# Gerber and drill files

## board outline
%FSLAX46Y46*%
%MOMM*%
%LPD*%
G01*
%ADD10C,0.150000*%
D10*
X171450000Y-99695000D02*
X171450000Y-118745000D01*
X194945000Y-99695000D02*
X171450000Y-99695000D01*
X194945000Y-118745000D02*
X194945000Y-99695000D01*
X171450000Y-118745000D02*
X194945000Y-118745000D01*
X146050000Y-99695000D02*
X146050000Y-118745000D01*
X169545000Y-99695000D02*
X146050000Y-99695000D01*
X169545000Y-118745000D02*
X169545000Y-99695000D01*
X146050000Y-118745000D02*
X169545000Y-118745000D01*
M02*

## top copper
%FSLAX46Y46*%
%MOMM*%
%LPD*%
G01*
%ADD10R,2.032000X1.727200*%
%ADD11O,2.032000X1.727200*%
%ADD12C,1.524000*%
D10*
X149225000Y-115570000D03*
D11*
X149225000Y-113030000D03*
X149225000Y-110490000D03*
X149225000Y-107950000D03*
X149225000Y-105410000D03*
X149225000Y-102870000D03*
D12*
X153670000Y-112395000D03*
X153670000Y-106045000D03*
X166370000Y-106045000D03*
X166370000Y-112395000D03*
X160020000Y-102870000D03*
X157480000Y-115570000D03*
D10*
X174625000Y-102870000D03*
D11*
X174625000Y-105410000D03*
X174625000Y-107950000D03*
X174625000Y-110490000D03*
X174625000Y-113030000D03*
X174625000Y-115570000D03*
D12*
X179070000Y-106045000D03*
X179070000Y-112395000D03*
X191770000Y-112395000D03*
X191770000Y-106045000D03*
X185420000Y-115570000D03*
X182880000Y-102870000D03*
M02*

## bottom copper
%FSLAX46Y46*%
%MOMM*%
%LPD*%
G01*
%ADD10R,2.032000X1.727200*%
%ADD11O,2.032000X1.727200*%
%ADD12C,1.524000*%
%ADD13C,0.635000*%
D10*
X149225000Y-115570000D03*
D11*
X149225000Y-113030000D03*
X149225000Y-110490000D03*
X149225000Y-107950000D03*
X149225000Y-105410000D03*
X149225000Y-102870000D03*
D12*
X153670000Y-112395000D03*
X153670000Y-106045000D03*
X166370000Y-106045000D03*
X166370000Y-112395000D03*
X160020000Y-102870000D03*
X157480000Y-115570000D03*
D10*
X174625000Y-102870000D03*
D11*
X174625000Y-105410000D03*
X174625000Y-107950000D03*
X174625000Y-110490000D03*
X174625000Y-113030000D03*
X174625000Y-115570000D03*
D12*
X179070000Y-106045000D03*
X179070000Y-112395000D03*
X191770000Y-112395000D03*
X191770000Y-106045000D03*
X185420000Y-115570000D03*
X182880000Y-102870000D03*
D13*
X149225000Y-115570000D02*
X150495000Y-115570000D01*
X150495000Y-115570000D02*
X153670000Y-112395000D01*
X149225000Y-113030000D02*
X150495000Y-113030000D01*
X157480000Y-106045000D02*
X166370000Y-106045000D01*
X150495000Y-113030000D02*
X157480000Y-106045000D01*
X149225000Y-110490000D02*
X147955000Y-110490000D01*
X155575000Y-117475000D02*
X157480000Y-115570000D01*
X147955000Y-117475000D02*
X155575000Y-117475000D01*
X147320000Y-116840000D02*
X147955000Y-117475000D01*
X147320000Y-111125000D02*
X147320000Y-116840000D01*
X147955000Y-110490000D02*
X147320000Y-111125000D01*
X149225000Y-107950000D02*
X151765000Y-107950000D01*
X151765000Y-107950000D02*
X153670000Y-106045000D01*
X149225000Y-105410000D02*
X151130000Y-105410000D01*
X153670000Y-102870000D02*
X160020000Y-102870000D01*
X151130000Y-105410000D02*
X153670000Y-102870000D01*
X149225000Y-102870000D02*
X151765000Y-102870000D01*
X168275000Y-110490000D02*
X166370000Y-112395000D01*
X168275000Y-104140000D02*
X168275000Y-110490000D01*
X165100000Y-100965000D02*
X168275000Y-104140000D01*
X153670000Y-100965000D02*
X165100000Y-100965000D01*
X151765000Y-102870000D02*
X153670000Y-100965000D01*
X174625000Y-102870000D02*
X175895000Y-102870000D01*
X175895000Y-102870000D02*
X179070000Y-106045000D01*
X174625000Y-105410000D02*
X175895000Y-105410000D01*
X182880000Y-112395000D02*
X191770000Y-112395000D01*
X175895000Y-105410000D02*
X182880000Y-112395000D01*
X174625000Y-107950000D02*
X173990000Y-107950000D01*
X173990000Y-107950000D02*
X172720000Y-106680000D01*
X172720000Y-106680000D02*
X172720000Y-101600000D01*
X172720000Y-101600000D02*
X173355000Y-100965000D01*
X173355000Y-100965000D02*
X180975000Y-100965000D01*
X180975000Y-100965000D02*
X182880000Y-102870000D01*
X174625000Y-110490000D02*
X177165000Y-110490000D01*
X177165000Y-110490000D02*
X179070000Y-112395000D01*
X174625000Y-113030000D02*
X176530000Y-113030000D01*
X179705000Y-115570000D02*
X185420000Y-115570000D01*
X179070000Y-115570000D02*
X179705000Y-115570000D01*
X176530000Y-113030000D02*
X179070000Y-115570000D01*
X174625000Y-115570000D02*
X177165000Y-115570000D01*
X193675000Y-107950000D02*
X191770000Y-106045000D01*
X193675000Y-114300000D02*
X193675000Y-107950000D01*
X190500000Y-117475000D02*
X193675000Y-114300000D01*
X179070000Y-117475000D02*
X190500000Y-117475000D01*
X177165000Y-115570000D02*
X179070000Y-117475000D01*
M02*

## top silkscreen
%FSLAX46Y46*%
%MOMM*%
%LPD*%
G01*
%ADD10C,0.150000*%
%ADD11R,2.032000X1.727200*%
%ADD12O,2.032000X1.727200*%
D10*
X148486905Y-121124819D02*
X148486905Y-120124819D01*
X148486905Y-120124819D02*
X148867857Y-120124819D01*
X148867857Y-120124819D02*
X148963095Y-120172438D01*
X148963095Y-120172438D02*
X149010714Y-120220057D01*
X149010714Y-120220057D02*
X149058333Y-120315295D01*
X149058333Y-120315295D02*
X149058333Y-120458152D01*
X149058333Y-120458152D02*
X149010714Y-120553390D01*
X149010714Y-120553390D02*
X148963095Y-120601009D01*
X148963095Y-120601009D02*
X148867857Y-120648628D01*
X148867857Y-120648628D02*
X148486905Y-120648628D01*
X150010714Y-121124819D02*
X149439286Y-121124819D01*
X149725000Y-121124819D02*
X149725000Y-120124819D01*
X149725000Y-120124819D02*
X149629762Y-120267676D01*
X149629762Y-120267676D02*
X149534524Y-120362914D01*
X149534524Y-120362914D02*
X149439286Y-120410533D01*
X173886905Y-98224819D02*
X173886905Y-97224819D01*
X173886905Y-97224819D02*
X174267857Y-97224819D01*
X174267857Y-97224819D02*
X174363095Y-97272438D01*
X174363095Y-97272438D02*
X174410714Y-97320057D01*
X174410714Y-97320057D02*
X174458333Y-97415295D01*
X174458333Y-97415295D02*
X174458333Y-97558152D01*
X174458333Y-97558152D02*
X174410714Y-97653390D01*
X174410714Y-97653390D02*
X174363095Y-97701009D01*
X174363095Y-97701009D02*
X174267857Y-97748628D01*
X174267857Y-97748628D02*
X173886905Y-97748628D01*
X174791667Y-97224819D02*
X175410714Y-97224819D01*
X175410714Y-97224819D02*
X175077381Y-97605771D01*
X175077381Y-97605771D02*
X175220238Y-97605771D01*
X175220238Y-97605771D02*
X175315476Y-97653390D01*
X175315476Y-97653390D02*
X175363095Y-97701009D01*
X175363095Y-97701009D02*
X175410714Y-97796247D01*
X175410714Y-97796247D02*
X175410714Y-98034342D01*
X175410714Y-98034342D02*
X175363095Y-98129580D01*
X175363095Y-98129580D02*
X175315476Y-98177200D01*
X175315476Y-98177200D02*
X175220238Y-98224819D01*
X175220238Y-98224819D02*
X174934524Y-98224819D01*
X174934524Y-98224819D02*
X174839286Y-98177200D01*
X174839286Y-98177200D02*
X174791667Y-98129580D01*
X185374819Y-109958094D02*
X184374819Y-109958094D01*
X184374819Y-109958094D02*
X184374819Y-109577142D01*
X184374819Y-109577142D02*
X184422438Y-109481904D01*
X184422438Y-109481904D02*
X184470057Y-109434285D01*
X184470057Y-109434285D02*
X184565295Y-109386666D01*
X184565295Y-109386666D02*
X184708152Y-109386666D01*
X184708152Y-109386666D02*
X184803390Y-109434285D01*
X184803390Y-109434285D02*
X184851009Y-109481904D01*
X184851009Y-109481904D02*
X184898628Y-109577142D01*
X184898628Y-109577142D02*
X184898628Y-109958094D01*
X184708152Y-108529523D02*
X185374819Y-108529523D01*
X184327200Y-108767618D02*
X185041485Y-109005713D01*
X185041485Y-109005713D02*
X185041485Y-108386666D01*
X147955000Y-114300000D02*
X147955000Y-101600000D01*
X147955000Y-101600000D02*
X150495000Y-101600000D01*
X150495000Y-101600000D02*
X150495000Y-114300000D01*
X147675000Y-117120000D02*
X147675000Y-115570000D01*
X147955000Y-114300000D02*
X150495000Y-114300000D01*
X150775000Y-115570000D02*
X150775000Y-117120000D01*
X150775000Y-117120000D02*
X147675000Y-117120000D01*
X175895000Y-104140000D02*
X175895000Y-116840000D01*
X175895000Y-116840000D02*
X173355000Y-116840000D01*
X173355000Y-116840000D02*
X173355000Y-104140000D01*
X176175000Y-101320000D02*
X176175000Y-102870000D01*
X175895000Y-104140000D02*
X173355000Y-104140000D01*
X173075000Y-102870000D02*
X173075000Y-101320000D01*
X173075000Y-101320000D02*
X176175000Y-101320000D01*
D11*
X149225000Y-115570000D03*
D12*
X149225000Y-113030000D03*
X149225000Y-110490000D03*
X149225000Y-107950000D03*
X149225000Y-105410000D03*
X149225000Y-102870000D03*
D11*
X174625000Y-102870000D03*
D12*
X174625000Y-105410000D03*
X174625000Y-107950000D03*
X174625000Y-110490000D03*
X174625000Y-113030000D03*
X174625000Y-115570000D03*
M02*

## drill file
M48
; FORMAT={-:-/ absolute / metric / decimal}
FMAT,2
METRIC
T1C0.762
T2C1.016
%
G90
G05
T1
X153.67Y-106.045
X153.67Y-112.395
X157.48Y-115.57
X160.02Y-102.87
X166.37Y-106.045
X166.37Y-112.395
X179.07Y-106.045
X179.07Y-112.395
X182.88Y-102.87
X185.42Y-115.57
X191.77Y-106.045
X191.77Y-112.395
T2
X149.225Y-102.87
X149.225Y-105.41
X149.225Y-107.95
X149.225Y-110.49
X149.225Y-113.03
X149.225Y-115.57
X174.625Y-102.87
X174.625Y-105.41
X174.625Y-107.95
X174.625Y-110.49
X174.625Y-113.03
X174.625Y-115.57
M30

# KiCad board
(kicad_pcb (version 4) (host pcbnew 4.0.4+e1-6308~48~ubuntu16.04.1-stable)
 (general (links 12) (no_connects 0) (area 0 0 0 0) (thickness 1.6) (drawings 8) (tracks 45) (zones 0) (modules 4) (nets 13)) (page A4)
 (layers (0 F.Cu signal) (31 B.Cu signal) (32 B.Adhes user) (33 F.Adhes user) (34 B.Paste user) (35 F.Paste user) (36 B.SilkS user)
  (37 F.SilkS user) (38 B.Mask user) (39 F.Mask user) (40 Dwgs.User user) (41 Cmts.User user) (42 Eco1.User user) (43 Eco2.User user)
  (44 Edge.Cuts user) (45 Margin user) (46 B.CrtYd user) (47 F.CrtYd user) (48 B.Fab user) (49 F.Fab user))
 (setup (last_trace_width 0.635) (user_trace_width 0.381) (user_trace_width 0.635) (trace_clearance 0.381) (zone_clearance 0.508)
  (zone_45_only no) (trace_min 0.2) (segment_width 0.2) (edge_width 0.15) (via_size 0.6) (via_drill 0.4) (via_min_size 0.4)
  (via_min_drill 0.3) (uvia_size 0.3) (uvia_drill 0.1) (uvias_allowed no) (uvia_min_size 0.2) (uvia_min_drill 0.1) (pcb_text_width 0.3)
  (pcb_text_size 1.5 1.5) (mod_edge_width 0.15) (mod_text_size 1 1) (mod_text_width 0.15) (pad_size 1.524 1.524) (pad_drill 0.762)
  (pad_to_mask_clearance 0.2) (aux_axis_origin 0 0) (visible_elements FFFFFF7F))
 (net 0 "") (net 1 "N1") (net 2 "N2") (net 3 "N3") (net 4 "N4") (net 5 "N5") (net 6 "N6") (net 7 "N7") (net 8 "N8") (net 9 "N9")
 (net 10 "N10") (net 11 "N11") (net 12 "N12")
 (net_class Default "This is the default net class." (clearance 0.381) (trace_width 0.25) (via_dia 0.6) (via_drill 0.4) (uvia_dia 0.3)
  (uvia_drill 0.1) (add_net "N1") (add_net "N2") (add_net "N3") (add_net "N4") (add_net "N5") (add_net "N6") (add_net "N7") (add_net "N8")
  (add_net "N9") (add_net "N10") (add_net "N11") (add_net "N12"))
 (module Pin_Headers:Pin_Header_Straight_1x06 (layer F.Cu) (at 149.225 115.57 180)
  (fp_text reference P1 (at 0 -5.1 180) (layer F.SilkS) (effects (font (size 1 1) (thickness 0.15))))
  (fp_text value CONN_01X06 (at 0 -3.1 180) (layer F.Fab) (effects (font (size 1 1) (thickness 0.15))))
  (fp_line (start 1.27 1.27) (end 1.27 13.97) (layer F.SilkS) (width 0.15))
  (fp_line (start 1.27 13.97) (end -1.27 13.97) (layer F.SilkS) (width 0.15))
  (fp_line (start -1.27 13.97) (end -1.27 1.27) (layer F.SilkS) (width 0.15))
  (fp_line (start 1.55 -1.55) (end 1.55 0) (layer F.SilkS) (width 0.15))
  (fp_line (start 1.27 1.27) (end -1.27 1.27) (layer F.SilkS) (width 0.15))
  (fp_line (start -1.55 0) (end -1.55 -1.55) (layer F.SilkS) (width 0.15))
  (fp_line (start -1.55 -1.55) (end 1.55 -1.55) (layer F.SilkS) (width 0.15))
  (pad 1 thru_hole rect (at 0 0 180) (size 2.032 1.7272) (drill 1.016) (layers *.Cu *.Mask F.SilkS) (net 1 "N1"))
  (pad 2 thru_hole oval (at 0 2.54 180) (size 2.032 1.7272) (drill 1.016) (layers *.Cu *.Mask F.SilkS) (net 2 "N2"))
  (pad 3 thru_hole oval (at 0 5.08 180) (size 2.032 1.7272) (drill 1.016) (layers *.Cu *.Mask F.SilkS) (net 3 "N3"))
  (pad 4 thru_hole oval (at 0 7.62 180) (size 2.032 1.7272) (drill 1.016) (layers *.Cu *.Mask F.SilkS) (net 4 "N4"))
  (pad 5 thru_hole oval (at 0 10.16 180) (size 2.032 1.7272) (drill 1.016) (layers *.Cu *.Mask F.SilkS) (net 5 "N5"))
  (pad 6 thru_hole oval (at 0 12.7 180) (size 2.032 1.7272) (drill 1.016) (layers *.Cu *.Mask F.SilkS) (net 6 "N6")))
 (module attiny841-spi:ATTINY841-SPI (layer B.Cu) (at 160.02 109.22 90)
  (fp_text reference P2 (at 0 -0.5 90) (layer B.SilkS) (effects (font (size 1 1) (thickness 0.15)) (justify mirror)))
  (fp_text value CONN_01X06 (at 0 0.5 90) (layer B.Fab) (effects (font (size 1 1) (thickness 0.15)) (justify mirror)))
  (pad 1 thru_hole circle (at -3.175 -6.35 90) (size 1.524 1.524) (drill 0.762) (layers *.Cu *.Mask) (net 1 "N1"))
  (pad 4 thru_hole circle (at 3.175 -6.35 90) (size 1.524 1.524) (drill 0.762) (layers *.Cu *.Mask) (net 4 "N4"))
  (pad 2 thru_hole circle (at 3.175 6.35 90) (size 1.524 1.524) (drill 0.762) (layers *.Cu *.Mask) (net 2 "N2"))
  (pad 6 thru_hole circle (at -3.175 6.35 90) (size 1.524 1.524) (drill 0.762) (layers *.Cu *.Mask) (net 6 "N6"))
  (pad 5 thru_hole circle (at 6.35 0 90) (size 1.524 1.524) (drill 0.762) (layers *.Cu *.Mask) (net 5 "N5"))
  (pad 3 thru_hole circle (at -6.35 -2.54 90) (size 1.524 1.524) (drill 0.762) (layers *.Cu *.Mask) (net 3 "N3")))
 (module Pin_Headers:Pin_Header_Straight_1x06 (layer F.Cu) (at 174.625 102.87)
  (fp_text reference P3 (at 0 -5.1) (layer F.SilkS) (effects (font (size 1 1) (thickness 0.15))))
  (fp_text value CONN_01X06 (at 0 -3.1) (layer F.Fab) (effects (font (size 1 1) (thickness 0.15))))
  (fp_line (start 1.27 1.27) (end 1.27 13.97) (layer F.SilkS) (width 0.15))
  (fp_line (start 1.27 13.97) (end -1.27 13.97) (layer F.SilkS) (width 0.15))
  (fp_line (start -1.27 13.97) (end -1.27 1.27) (layer F.SilkS) (width 0.15))
  (fp_line (start 1.55 -1.55) (end 1.55 0) (layer F.SilkS) (width 0.15))
  (fp_line (start 1.27 1.27) (end -1.27 1.27) (layer F.SilkS) (width 0.15))
  (fp_line (start -1.55 0) (end -1.55 -1.55) (layer F.SilkS) (width 0.15))
  (fp_line (start -1.55 -1.55) (end 1.55 -1.55) (layer F.SilkS) (width 0.15))
  (pad 1 thru_hole rect (at 0 0) (size 2.032 1.7272) (drill 1.016) (layers *.Cu *.Mask F.SilkS) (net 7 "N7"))
  (pad 2 thru_hole oval (at 0 2.54) (size 2.032 1.7272) (drill 1.016) (layers *.Cu *.Mask F.SilkS) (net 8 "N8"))
  (pad 3 thru_hole oval (at 0 5.08) (size 2.032 1.7272) (drill 1.016) (layers *.Cu *.Mask F.SilkS) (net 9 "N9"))
  (pad 4 thru_hole oval (at 0 7.62) (size 2.032 1.7272) (drill 1.016) (layers *.Cu *.Mask F.SilkS) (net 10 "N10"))
  (pad 5 thru_hole oval (at 0 10.16) (size 2.032 1.7272) (drill 1.016) (layers *.Cu *.Mask F.SilkS) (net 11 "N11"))
  (pad 6 thru_hole oval (at 0 12.7) (size 2.032 1.7272) (drill 1.016) (layers *.Cu *.Mask F.SilkS) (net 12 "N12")))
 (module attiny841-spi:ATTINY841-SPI (layer F.Cu) (at 185.42 109.22 270)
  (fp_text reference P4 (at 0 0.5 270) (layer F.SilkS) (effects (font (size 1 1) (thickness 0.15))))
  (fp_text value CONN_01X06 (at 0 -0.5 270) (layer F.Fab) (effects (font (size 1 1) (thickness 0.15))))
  (pad 1 thru_hole circle (at -3.175 6.35 270) (size 1.524 1.524) (drill 0.762) (layers *.Cu *.Mask) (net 7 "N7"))
  (pad 4 thru_hole circle (at 3.175 6.35 270) (size 1.524 1.524) (drill 0.762) (layers *.Cu *.Mask) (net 10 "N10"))
  (pad 2 thru_hole circle (at 3.175 -6.35 270) (size 1.524 1.524) (drill 0.762) (layers *.Cu *.Mask) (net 8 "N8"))
  (pad 6 thru_hole circle (at -3.175 -6.35 270) (size 1.524 1.524) (drill 0.762) (layers *.Cu *.Mask) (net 12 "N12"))
  (pad 5 thru_hole circle (at 6.35 0 270) (size 1.524 1.524) (drill 0.762) (layers *.Cu *.Mask) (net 11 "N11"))
  (pad 3 thru_hole circle (at -6.35 2.54 270) (size 1.524 1.524) (drill 0.762) (layers *.Cu *.Mask) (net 9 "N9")))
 (gr_line (start 171.45 99.695) (end 171.45 118.745) (angle 90) (layer Edge.Cuts) (width 0.15))
 (gr_line (start 194.945 99.695) (end 171.45 99.695) (angle 90) (layer Edge.Cuts) (width 0.15))
 (gr_line (start 194.945 118.745) (end 194.945 99.695) (angle 90) (layer Edge.Cuts) (width 0.15))
 (gr_line (start 171.45 118.745) (end 194.945 118.745) (angle 90) (layer Edge.Cuts) (width 0.15))
 (gr_line (start 146.05 99.695) (end 146.05 118.745) (angle 90) (layer Edge.Cuts) (width 0.15))
 (gr_line (start 169.545 99.695) (end 146.05 99.695) (angle 90) (layer Edge.Cuts) (width 0.15))
 (gr_line (start 169.545 118.745) (end 169.545 99.695) (angle 90) (layer Edge.Cuts) (width 0.15))
 (gr_line (start 146.05 118.745) (end 169.545 118.745) (angle 90) (layer Edge.Cuts) (width 0.15))
 (segment (start 149.225 115.57) (end 150.495 115.57) (width 0.635) (layer B.Cu) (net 1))
 (segment (start 150.495 115.57) (end 153.67 112.395) (width 0.635) (layer B.Cu) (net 1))
 (segment (start 149.225 113.03) (end 150.495 113.03) (width 0.635) (layer B.Cu) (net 2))
 (segment (start 157.48 106.045) (end 166.37 106.045) (width 0.635) (layer B.Cu) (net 2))
 (segment (start 150.495 113.03) (end 157.48 106.045) (width 0.635) (layer B.Cu) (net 2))
 (segment (start 149.225 110.49) (end 147.955 110.49) (width 0.635) (layer B.Cu) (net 3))
 (segment (start 155.575 117.475) (end 157.48 115.57) (width 0.635) (layer B.Cu) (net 3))
 (segment (start 147.955 117.475) (end 155.575 117.475) (width 0.635) (layer B.Cu) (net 3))
 (segment (start 147.32 116.84) (end 147.955 117.475) (width 0.635) (layer B.Cu) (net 3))
 (segment (start 147.32 111.125) (end 147.32 116.84) (width 0.635) (layer B.Cu) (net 3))
 (segment (start 147.955 110.49) (end 147.32 111.125) (width 0.635) (layer B.Cu) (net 3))
 (segment (start 149.225 107.95) (end 151.765 107.95) (width 0.635) (layer B.Cu) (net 4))
 (segment (start 151.765 107.95) (end 153.67 106.045) (width 0.635) (layer B.Cu) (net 4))
 (segment (start 149.225 105.41) (end 151.13 105.41) (width 0.635) (layer B.Cu) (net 5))
 (segment (start 153.67 102.87) (end 160.02 102.87) (width 0.635) (layer B.Cu) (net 5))
 (segment (start 151.13 105.41) (end 153.67 102.87) (width 0.635) (layer B.Cu) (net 5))
 (segment (start 149.225 102.87) (end 151.765 102.87) (width 0.635) (layer B.Cu) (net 6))
 (segment (start 168.275 110.49) (end 166.37 112.395) (width 0.635) (layer B.Cu) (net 6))
 (segment (start 168.275 104.14) (end 168.275 110.49) (width 0.635) (layer B.Cu) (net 6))
 (segment (start 165.1 100.965) (end 168.275 104.14) (width 0.635) (layer B.Cu) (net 6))
 (segment (start 153.67 100.965) (end 165.1 100.965) (width 0.635) (layer B.Cu) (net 6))
 (segment (start 151.765 102.87) (end 153.67 100.965) (width 0.635) (layer B.Cu) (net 6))
 (segment (start 174.625 102.87) (end 175.895 102.87) (width 0.635) (layer B.Cu) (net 7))
 (segment (start 175.895 102.87) (end 179.07 106.045) (width 0.635) (layer B.Cu) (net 7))
 (segment (start 174.625 105.41) (end 175.895 105.41) (width 0.635) (layer B.Cu) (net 8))
 (segment (start 182.88 112.395) (end 191.77 112.395) (width 0.635) (layer B.Cu) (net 8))
 (segment (start 175.895 105.41) (end 182.88 112.395) (width 0.635) (layer B.Cu) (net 8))
 (segment (start 174.625 107.95) (end 173.99 107.95) (width 0.635) (layer B.Cu) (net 9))
 (segment (start 173.99 107.95) (end 172.72 106.68) (width 0.635) (layer B.Cu) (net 9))
 (segment (start 172.72 106.68) (end 172.72 101.6) (width 0.635) (layer B.Cu) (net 9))
 (segment (start 172.72 101.6) (end 173.355 100.965) (width 0.635) (layer B.Cu) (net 9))
 (segment (start 173.355 100.965) (end 180.975 100.965) (width 0.635) (layer B.Cu) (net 9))
 (segment (start 180.975 100.965) (end 182.88 102.87) (width 0.635) (layer B.Cu) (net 9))
 (segment (start 174.625 110.49) (end 177.165 110.49) (width 0.635) (layer B.Cu) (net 10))
 (segment (start 177.165 110.49) (end 179.07 112.395) (width 0.635) (layer B.Cu) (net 10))
 (segment (start 174.625 113.03) (end 176.53 113.03) (width 0.635) (layer B.Cu) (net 11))
 (segment (start 179.705 115.57) (end 185.42 115.57) (width 0.635) (layer B.Cu) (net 11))
 (segment (start 179.07 115.57) (end 179.705 115.57) (width 0.635) (layer B.Cu) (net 11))
 (segment (start 176.53 113.03) (end 179.07 115.57) (width 0.635) (layer B.Cu) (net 11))
 (segment (start 174.625 115.57) (end 177.165 115.57) (width 0.635) (layer B.Cu) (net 12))
 (segment (start 193.675 107.95) (end 191.77 106.045) (width 0.635) (layer B.Cu) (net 12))
 (segment (start 193.675 114.3) (end 193.675 107.95) (width 0.635) (layer B.Cu) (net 12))
 (segment (start 190.5 117.475) (end 193.675 114.3) (width 0.635) (layer B.Cu) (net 12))
 (segment (start 179.07 117.475) (end 190.5 117.475) (width 0.635) (layer B.Cu) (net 12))
 (segment (start 177.165 115.57) (end 179.07 117.475) (width 0.635) (layer B.Cu) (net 12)))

